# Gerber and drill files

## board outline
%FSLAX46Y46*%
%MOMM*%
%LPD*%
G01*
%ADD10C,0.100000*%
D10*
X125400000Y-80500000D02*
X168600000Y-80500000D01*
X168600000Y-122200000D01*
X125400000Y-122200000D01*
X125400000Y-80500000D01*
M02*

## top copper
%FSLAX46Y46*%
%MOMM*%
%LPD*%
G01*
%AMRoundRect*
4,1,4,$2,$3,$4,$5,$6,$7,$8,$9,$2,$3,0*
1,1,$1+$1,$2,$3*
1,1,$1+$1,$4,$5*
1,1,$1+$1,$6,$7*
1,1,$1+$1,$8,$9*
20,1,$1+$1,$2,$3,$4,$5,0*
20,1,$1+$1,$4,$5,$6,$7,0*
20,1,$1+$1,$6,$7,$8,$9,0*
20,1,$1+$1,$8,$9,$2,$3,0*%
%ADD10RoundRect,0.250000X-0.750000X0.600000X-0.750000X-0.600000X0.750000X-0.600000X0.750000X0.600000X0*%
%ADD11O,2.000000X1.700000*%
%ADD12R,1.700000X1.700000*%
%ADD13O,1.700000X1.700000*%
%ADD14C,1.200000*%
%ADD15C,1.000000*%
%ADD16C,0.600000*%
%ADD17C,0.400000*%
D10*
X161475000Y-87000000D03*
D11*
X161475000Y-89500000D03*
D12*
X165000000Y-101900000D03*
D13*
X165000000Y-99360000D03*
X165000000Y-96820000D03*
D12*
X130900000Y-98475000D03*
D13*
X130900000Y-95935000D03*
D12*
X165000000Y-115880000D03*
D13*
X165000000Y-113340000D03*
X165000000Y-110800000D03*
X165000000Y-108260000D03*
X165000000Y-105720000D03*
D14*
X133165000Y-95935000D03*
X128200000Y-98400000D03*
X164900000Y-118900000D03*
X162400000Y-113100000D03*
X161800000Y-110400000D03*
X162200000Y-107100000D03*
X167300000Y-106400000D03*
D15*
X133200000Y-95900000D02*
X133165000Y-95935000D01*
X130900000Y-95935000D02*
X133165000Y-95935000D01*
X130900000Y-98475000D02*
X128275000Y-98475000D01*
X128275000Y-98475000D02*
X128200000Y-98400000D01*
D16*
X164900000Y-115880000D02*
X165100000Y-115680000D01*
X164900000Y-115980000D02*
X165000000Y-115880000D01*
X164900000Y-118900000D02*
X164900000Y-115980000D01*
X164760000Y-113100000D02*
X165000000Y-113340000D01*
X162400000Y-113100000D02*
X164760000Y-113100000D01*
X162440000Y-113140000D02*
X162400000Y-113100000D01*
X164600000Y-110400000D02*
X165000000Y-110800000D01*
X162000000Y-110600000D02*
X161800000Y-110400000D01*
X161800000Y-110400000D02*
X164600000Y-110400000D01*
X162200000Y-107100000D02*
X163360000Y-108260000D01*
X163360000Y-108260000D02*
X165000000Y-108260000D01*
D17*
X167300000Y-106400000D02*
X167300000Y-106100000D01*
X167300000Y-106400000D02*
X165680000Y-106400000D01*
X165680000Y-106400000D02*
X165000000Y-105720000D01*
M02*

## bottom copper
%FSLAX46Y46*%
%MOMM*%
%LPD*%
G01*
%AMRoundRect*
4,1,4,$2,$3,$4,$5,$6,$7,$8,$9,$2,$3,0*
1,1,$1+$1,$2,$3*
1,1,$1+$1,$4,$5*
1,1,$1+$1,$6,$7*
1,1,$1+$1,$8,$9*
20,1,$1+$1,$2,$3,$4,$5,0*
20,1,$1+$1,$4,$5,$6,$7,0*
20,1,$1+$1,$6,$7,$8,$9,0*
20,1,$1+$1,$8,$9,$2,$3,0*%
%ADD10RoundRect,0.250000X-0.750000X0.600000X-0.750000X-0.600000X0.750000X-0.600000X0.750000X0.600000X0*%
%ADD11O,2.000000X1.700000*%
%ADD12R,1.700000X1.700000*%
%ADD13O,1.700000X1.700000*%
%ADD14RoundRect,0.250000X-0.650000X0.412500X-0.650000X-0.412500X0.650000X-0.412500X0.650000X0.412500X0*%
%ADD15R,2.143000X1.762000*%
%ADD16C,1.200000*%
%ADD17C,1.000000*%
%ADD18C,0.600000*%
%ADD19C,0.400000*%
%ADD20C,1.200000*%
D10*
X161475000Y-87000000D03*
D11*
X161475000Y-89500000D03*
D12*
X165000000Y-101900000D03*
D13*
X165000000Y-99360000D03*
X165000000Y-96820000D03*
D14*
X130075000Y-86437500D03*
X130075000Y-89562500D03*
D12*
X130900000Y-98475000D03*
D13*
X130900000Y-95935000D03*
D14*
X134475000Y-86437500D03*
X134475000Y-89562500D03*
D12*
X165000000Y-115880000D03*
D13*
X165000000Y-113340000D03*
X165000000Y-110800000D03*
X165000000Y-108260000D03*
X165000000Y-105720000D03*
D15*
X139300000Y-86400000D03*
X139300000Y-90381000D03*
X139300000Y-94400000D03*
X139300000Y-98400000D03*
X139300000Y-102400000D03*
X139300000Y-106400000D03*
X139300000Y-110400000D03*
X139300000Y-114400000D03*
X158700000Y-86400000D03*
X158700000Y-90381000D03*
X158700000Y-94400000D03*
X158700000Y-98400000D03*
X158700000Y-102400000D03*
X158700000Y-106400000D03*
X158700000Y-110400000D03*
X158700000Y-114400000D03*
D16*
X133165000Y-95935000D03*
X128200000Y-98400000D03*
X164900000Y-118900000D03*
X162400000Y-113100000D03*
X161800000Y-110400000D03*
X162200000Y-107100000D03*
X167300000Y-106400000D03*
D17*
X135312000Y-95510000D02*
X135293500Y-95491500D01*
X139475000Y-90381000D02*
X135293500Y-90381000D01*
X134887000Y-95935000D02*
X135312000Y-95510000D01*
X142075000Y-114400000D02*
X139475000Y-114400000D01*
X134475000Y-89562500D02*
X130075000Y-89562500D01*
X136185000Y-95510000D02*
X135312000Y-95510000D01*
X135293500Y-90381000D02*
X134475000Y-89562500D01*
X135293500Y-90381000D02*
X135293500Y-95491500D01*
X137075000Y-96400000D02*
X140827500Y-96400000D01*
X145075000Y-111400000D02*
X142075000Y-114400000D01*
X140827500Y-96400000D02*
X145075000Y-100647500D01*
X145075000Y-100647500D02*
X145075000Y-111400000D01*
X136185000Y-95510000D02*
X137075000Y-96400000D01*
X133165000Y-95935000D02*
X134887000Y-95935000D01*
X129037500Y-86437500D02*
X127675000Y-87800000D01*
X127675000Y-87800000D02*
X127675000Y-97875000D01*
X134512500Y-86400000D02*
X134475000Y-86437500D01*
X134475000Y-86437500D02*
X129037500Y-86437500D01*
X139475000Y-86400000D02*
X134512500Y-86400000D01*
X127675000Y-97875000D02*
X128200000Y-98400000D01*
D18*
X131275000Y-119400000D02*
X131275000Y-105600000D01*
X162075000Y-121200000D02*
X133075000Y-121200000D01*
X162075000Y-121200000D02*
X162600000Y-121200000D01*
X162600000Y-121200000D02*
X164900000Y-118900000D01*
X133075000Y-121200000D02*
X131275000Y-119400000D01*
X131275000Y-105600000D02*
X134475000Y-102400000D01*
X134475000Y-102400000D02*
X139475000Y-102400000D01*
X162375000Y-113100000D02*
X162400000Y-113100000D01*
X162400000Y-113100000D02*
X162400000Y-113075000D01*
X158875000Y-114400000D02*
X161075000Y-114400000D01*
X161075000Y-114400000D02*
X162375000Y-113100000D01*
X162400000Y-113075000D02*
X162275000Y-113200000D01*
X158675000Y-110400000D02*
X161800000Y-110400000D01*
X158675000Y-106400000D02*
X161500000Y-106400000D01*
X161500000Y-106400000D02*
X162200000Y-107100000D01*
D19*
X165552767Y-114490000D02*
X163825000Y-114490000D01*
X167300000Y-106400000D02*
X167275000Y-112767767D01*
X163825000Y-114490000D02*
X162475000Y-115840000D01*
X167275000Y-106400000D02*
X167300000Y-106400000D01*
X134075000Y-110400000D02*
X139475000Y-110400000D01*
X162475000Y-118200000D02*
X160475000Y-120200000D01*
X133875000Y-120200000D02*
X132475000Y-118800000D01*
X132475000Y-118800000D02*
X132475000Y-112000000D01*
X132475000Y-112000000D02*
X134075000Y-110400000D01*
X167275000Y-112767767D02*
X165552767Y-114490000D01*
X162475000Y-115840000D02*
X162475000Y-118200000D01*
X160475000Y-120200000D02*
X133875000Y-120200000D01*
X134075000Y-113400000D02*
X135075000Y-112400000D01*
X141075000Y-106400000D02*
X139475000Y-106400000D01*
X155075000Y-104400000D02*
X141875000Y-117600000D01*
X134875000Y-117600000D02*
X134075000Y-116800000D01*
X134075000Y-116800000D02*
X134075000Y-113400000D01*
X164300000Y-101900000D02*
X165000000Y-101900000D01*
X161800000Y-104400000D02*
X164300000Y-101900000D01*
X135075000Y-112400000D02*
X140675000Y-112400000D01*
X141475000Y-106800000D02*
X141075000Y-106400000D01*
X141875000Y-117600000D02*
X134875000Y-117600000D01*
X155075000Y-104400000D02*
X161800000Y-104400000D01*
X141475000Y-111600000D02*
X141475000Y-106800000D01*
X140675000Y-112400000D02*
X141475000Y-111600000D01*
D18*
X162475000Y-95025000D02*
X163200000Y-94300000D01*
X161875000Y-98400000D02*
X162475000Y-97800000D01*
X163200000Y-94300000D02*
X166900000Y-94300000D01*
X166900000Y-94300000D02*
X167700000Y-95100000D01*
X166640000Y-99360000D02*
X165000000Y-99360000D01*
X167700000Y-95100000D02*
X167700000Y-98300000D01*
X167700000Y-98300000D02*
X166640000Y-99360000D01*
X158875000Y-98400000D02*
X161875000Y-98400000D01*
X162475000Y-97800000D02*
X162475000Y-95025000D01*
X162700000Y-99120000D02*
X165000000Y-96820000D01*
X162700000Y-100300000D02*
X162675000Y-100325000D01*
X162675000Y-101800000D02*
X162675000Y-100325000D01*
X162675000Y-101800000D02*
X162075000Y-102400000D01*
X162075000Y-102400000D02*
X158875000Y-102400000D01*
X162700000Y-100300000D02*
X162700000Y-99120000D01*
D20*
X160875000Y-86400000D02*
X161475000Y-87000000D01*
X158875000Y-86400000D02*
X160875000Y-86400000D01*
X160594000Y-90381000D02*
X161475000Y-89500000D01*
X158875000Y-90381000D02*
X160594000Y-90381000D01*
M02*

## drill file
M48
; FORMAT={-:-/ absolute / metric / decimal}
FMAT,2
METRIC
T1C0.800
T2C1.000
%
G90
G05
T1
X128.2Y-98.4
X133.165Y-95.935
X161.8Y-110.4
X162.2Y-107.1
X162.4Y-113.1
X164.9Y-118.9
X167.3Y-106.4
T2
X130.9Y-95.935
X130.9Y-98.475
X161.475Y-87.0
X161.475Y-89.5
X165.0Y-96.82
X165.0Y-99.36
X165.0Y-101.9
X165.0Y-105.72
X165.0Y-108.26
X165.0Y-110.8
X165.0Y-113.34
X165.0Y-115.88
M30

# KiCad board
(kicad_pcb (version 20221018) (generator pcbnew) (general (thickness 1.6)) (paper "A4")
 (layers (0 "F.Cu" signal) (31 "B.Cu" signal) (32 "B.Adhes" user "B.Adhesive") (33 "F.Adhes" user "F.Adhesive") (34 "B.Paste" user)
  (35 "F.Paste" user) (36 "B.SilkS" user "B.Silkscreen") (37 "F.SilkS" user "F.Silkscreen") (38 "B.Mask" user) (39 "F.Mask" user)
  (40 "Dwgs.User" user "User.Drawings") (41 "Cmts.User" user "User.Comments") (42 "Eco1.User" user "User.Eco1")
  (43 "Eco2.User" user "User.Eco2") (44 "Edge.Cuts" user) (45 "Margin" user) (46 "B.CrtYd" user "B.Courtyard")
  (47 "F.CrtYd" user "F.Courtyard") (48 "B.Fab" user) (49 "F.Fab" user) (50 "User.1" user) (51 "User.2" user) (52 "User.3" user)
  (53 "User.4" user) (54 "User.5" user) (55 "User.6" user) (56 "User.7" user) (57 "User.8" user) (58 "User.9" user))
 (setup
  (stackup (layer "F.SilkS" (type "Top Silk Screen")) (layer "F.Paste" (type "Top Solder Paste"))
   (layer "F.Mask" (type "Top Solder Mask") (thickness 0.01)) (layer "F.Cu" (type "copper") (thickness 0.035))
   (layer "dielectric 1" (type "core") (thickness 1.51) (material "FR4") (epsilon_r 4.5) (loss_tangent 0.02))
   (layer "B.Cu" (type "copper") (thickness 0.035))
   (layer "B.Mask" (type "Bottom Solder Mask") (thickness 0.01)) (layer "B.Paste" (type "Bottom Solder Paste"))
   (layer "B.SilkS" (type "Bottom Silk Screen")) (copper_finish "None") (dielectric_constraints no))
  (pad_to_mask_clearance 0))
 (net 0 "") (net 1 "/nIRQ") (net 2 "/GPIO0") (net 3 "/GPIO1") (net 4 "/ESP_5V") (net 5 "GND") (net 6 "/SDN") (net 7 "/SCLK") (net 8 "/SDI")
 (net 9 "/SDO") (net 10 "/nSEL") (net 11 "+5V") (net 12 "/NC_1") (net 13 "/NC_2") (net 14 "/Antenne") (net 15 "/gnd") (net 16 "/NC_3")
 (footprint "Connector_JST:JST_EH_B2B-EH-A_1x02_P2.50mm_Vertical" (layer "F.Cu") (at 161.475 87 -90)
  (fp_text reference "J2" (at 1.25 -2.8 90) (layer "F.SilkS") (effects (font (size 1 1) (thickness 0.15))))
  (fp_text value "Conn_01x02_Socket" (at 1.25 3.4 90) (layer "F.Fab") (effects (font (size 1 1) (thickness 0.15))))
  (pad "1" thru_hole roundrect (at 0 0 270) (size 1.7 2) (drill 1) (layers "*.Cu" "*.Mask") (roundrect_rratio 0.1470588235))
  (pad "2" thru_hole oval (at 2.5 0 270) (size 1.7 2) (drill 1) (layers "*.Cu" "*.Mask")))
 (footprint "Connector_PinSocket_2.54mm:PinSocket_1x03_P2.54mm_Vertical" (layer "F.Cu") (at 165 101.9 180)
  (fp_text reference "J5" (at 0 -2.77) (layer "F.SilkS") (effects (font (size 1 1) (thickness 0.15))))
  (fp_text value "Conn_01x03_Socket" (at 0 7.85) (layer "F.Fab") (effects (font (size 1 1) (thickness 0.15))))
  (pad "1" thru_hole rect (at 0 0 180) (size 1.7 1.7) (drill 1) (layers "*.Cu" "*.Mask") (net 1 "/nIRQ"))
  (pad "2" thru_hole oval (at 0 2.54 180) (size 1.7 1.7) (drill 1) (layers "*.Cu" "*.Mask") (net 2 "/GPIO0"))
  (pad "3" thru_hole oval (at 0 5.08 180) (size 1.7 1.7) (drill 1) (layers "*.Cu" "*.Mask") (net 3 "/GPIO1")))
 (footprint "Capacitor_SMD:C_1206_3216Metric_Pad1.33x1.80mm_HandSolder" (layer "B.Cu") (at 130.075 88 -90)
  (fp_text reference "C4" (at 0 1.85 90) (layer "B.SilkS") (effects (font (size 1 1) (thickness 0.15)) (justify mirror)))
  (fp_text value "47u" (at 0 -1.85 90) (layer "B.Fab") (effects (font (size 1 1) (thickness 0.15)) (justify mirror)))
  (pad "1" smd roundrect (at -1.5625 0 270) (size 1.325 1.8) (layers "B.Cu" "B.Paste" "B.Mask") (roundrect_rratio 0.1886792453))
  (pad "2" smd roundrect (at 1.5625 0 270) (size 1.325 1.8) (layers "B.Cu" "B.Paste" "B.Mask") (roundrect_rratio 0.1886792453)))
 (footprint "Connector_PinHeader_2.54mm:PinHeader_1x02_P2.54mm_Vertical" (layer "B.Cu") (at 130.9 98.475)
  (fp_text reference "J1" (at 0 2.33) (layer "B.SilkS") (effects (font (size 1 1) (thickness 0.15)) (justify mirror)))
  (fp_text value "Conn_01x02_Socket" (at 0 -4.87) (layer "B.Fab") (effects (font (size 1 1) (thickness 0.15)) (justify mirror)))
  (pad "1" thru_hole rect (at 0 0) (size 1.7 1.7) (drill 1) (layers "*.Cu" "*.Mask") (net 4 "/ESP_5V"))
  (pad "2" thru_hole oval (at 0 -2.54) (size 1.7 1.7) (drill 1) (layers "*.Cu" "*.Mask") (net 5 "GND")))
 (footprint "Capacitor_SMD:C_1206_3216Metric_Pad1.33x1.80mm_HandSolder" (layer "B.Cu") (at 134.475 88 -90)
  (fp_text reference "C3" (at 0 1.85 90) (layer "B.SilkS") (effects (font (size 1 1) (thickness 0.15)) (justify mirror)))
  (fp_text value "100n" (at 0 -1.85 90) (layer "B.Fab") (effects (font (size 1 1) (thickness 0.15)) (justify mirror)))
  (pad "1" smd roundrect (at -1.5625 0 270) (size 1.325 1.8) (layers "B.Cu" "B.Paste" "B.Mask") (roundrect_rratio 0.1886792453))
  (pad "2" smd roundrect (at 1.5625 0 270) (size 1.325 1.8) (layers "B.Cu" "B.Paste" "B.Mask") (roundrect_rratio 0.1886792453)))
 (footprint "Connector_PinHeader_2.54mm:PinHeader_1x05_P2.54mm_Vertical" (layer "B.Cu") (at 165 115.88)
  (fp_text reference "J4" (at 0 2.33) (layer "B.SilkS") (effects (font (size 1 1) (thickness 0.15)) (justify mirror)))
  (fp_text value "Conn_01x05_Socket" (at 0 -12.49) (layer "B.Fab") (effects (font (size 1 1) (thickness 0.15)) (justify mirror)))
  (pad "1" thru_hole rect (at 0 0) (size 1.7 1.7) (drill 1) (layers "*.Cu" "*.Mask") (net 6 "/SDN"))
  (pad "2" thru_hole oval (at 0 -2.54) (size 1.7 1.7) (drill 1) (layers "*.Cu" "*.Mask") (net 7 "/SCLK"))
  (pad "3" thru_hole oval (at 0 -5.08) (size 1.7 1.7) (drill 1) (layers "*.Cu" "*.Mask") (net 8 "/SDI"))
  (pad "4" thru_hole oval (at 0 -7.62) (size 1.7 1.7) (drill 1) (layers "*.Cu" "*.Mask") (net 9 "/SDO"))
  (pad "5" thru_hole oval (at 0 -10.16) (size 1.7 1.7) (drill 1) (layers "*.Cu" "*.Mask") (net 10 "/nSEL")))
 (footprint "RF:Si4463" (layer "B.Cu") (at 149 100.4 -90)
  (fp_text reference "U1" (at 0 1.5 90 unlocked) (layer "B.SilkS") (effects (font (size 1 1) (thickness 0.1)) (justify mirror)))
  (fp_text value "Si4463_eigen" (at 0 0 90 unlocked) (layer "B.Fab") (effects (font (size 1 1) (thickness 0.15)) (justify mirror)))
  (pad "1" smd rect (at -14 9.7 180) (size 2.143 1.762) (layers "B.Cu" "B.Paste" "B.Mask") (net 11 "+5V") (thermal_bridge_angle 45))
  (pad "2" smd rect (at -10.019 9.7 180) (size 2.143 1.762) (layers "B.Cu" "B.Paste" "B.Mask") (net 5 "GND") (thermal_bridge_angle 45))
  (pad "3" smd rect (at -6 9.7 180) (size 2.143 1.762) (layers "B.Cu" "B.Paste" "B.Mask") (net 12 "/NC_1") (thermal_bridge_angle 45))
  (pad "4" smd rect (at -2 9.7 180) (size 2.143 1.762) (layers "B.Cu" "B.Paste" "B.Mask") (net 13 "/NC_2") (thermal_bridge_angle 45))
  (pad "5" smd rect (at 2 9.7 180) (size 2.143 1.762) (layers "B.Cu" "B.Paste" "B.Mask") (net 6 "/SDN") (thermal_bridge_angle 45))
  (pad "6" smd rect (at 6 9.7 180) (size 2.143 1.762) (layers "B.Cu" "B.Paste" "B.Mask") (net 1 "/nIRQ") (thermal_bridge_angle 45))
  (pad "7" smd rect (at 10 9.7 180) (size 2.143 1.762) (layers "B.Cu" "B.Paste" "B.Mask") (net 10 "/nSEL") (thermal_bridge_angle 45))
  (pad "8" smd rect (at 14 9.7 180) (size 2.143 1.762) (layers "B.Cu" "B.Paste" "B.Mask") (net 5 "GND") (thermal_bridge_angle 45))
  (pad "9" smd rect (at -14 -9.7 180) (size 2.143 1.762) (layers "B.Cu" "B.Paste" "B.Mask") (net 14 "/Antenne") (thermal_bridge_angle 45))
  (pad "10" smd rect (at -10.019 -9.7 180) (size 2.143 1.762) (layers "B.Cu" "B.Paste" "B.Mask") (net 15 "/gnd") (thermal_bridge_angle 45))
  (pad "11" smd rect (at -6 -9.7 180) (size 2.143 1.762) (layers "B.Cu" "B.Paste" "B.Mask") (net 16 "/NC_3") (thermal_bridge_angle 45))
  (pad "12" smd rect (at -2 -9.7 180) (size 2.143 1.762) (layers "B.Cu" "B.Paste" "B.Mask") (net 2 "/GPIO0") (thermal_bridge_angle 45))
  (pad "13" smd rect (at 2 -9.7 180) (size 2.143 1.762) (layers "B.Cu" "B.Paste" "B.Mask") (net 3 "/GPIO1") (thermal_bridge_angle 45))
  (pad "14" smd rect (at 6 -9.7 180) (size 2.143 1.762) (layers "B.Cu" "B.Paste" "B.Mask") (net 9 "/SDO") (thermal_bridge_angle 45))
  (pad "15" smd rect (at 10 -9.7 180) (size 2.143 1.762) (layers "B.Cu" "B.Paste" "B.Mask") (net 8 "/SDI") (thermal_bridge_angle 45))
  (pad "16" smd rect (at 14 -9.7 180) (size 2.143 1.762) (layers "B.Cu" "B.Paste" "B.Mask") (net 7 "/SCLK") (thermal_bridge_angle 45)))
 (gr_rect (start 125.4 80.5) (end 168.6 122.2) (stroke (width 0.1) (type default)) (fill none) (layer "Edge.Cuts"))
 (segment (start 133.2 95.9) (end 133.165 95.935) (width 1) (layer "F.Cu") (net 5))
 (segment (start 130.9 95.935) (end 133.165 95.935) (width 1) (layer "F.Cu") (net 5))
 (via (at 133.165 95.935) (size 1.2) (drill 0.8) (layers "F.Cu" "B.Cu") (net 5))
 (segment (start 135.312 95.51) (end 135.2935 95.4915) (width 1) (layer "B.Cu") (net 5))
 (segment (start 139.475 90.381) (end 135.2935 90.381) (width 1) (layer "B.Cu") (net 5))
 (segment (start 134.887 95.935) (end 135.312 95.51) (width 1) (layer "B.Cu") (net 5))
 (segment (start 142.075 114.4) (end 139.475 114.4) (width 1) (layer "B.Cu") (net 5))
 (segment (start 134.475 89.5625) (end 130.075 89.5625) (width 1) (layer "B.Cu") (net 5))
 (segment (start 136.185 95.51) (end 135.312 95.51) (width 1) (layer "B.Cu") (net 5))
 (segment (start 135.2935 90.381) (end 134.475 89.5625) (width 1) (layer "B.Cu") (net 5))
 (segment (start 135.2935 90.381) (end 135.2935 95.4915) (width 1) (layer "B.Cu") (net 5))
 (segment (start 137.075 96.4) (end 140.8275 96.4) (width 1) (layer "B.Cu") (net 5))
 (segment (start 145.075 111.4) (end 142.075 114.4) (width 1) (layer "B.Cu") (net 5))
 (segment (start 140.8275 96.4) (end 145.075 100.6475) (width 1) (layer "B.Cu") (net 5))
 (segment (start 145.075 100.6475) (end 145.075 111.4) (width 1) (layer "B.Cu") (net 5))
 (segment (start 136.185 95.51) (end 137.075 96.4) (width 1) (layer "B.Cu") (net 5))
 (segment (start 133.165 95.935) (end 134.887 95.935) (width 1) (layer "B.Cu") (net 5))
 (segment (start 130.9 98.475) (end 128.275 98.475) (width 1) (layer "F.Cu") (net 4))
 (segment (start 128.275 98.475) (end 128.2 98.4) (width 1) (layer "F.Cu") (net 4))
 (via (at 128.2 98.4) (size 1.2) (drill 0.8) (layers "F.Cu" "B.Cu") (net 4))
 (segment (start 129.0375 86.4375) (end 127.675 87.8) (width 1) (layer "B.Cu") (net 4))
 (segment (start 127.675 87.8) (end 127.675 97.875) (width 1) (layer "B.Cu") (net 4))
 (segment (start 134.5125 86.4) (end 134.475 86.4375) (width 1) (layer "B.Cu") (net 4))
 (segment (start 134.475 86.4375) (end 129.0375 86.4375) (width 1) (layer "B.Cu") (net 4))
 (segment (start 139.475 86.4) (end 134.5125 86.4) (width 1) (layer "B.Cu") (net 4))
 (segment (start 127.675 97.875) (end 128.2 98.4) (width 1) (layer "B.Cu") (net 4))
 (segment (start 164.9 115.88) (end 165.1 115.68) (width 0.6) (layer "F.Cu") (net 6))
 (segment (start 164.9 115.98) (end 165 115.88) (width 0.6) (layer "F.Cu") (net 6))
 (segment (start 164.9 118.9) (end 164.9 115.98) (width 0.6) (layer "F.Cu") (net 6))
 (via (at 164.9 118.9) (size 1.2) (drill 0.8) (layers "F.Cu" "B.Cu") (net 6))
 (segment (start 131.275 119.4) (end 131.275 105.6) (width 0.6) (layer "B.Cu") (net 6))
 (segment (start 162.075 121.2) (end 133.075 121.2) (width 0.6) (layer "B.Cu") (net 6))
 (segment (start 162.075 121.2) (end 162.6 121.2) (width 0.6) (layer "B.Cu") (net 6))
 (segment (start 162.6 121.2) (end 164.9 118.9) (width 0.6) (layer "B.Cu") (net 6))
 (segment (start 133.075 121.2) (end 131.275 119.4) (width 0.6) (layer "B.Cu") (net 6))
 (segment (start 131.275 105.6) (end 134.475 102.4) (width 0.6) (layer "B.Cu") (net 6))
 (segment (start 134.475 102.4) (end 139.475 102.4) (width 0.6) (layer "B.Cu") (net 6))
 (segment (start 164.76 113.1) (end 165 113.34) (width 0.6) (layer "F.Cu") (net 7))
 (segment (start 162.4 113.1) (end 164.76 113.1) (width 0.6) (layer "F.Cu") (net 7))
 (segment (start 162.44 113.14) (end 162.4 113.1) (width 0.6) (layer "F.Cu") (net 7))
 (via (at 162.4 113.1) (size 1.2) (drill 0.8) (layers "F.Cu" "B.Cu") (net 7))
 (segment (start 162.375 113.1) (end 162.4 113.1) (width 0.6) (layer "B.Cu") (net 7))
 (segment (start 162.4 113.1) (end 162.4 113.075) (width 0.6) (layer "B.Cu") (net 7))
 (segment (start 158.875 114.4) (end 161.075 114.4) (width 0.6) (layer "B.Cu") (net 7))
 (segment (start 161.075 114.4) (end 162.375 113.1) (width 0.6) (layer "B.Cu") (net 7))
 (segment (start 162.4 113.075) (end 162.275 113.2) (width 0.6) (layer "B.Cu") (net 7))
 (segment (start 164.6 110.4) (end 165 110.8) (width 0.6) (layer "F.Cu") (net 8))
 (segment (start 162 110.6) (end 161.8 110.4) (width 0.6) (layer "F.Cu") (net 8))
 (segment (start 161.8 110.4) (end 164.6 110.4) (width 0.6) (layer "F.Cu") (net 8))
 (via (at 161.8 110.4) (size 1.2) (drill 0.8) (layers "F.Cu" "B.Cu") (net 8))
 (segment (start 158.675 110.4) (end 161.8 110.4) (width 0.6) (layer "B.Cu") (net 8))
 (segment (start 162.2 107.1) (end 163.36 108.26) (width 0.6) (layer "F.Cu") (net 9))
 (segment (start 163.36 108.26) (end 165 108.26) (width 0.6) (layer "F.Cu") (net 9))
 (via (at 162.2 107.1) (size 1.2) (drill 0.8) (layers "F.Cu" "B.Cu") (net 9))
 (segment (start 158.675 106.4) (end 161.5 106.4) (width 0.6) (layer "B.Cu") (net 9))
 (segment (start 161.5 106.4) (end 162.2 107.1) (width 0.6) (layer "B.Cu") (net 9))
 (segment (start 167.3 106.4) (end 167.3 106.1) (width 0.4) (layer "F.Cu") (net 10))
 (segment (start 167.3 106.4) (end 165.68 106.4) (width 0.4) (layer "F.Cu") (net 10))
 (segment (start 165.68 106.4) (end 165 105.72) (width 0.4) (layer "F.Cu") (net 10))
 (via (at 167.3 106.4) (size 1.2) (drill 0.8) (layers "F.Cu" "B.Cu") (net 10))
 (segment (start 165.552767 114.49) (end 163.825 114.49) (width 0.4) (layer "B.Cu") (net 10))
 (segment (start 167.3 106.4) (end 167.275 112.767767) (width 0.4) (layer "B.Cu") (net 10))
 (segment (start 163.825 114.49) (end 162.475 115.84) (width 0.4) (layer "B.Cu") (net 10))
 (segment (start 167.275 106.4) (end 167.3 106.4) (width 0.4) (layer "B.Cu") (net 10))
 (segment (start 134.075 110.4) (end 139.475 110.4) (width 0.4) (layer "B.Cu") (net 10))
 (segment (start 162.475 118.2) (end 160.475 120.2) (width 0.4) (layer "B.Cu") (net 10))
 (segment (start 133.875 120.2) (end 132.475 118.8) (width 0.4) (layer "B.Cu") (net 10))
 (segment (start 132.475 118.8) (end 132.475 112) (width 0.4) (layer "B.Cu") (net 10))
 (segment (start 132.475 112) (end 134.075 110.4) (width 0.4) (layer "B.Cu") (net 10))
 (segment (start 167.275 112.767767) (end 165.552767 114.49) (width 0.4) (layer "B.Cu") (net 10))
 (segment (start 162.475 115.84) (end 162.475 118.2) (width 0.4) (layer "B.Cu") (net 10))
 (segment (start 160.475 120.2) (end 133.875 120.2) (width 0.4) (layer "B.Cu") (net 10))
 (segment (start 134.075 113.4) (end 135.075 112.4) (width 0.4) (layer "B.Cu") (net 1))
 (segment (start 141.075 106.4) (end 139.475 106.4) (width 0.4) (layer "B.Cu") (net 1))
 (segment (start 155.075 104.4) (end 141.875 117.6) (width 0.4) (layer "B.Cu") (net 1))
 (segment (start 134.875 117.6) (end 134.075 116.8) (width 0.4) (layer "B.Cu") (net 1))
 (segment (start 134.075 116.8) (end 134.075 113.4) (width 0.4) (layer "B.Cu") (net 1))
 (segment (start 164.3 101.9) (end 165 101.9) (width 0.4) (layer "B.Cu") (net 1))
 (segment (start 161.8 104.4) (end 164.3 101.9) (width 0.4) (layer "B.Cu") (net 1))
 (segment (start 135.075 112.4) (end 140.675 112.4) (width 0.4) (layer "B.Cu") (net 1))
 (segment (start 141.475 106.8) (end 141.075 106.4) (width 0.4) (layer "B.Cu") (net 1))
 (segment (start 141.875 117.6) (end 134.875 117.6) (width 0.4) (layer "B.Cu") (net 1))
 (segment (start 155.075 104.4) (end 161.8 104.4) (width 0.4) (layer "B.Cu") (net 1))
 (segment (start 141.475 111.6) (end 141.475 106.8) (width 0.4) (layer "B.Cu") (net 1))
 (segment (start 140.675 112.4) (end 141.475 111.6) (width 0.4) (layer "B.Cu") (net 1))
 (segment (start 162.475 95.025) (end 163.2 94.3) (width 0.6) (layer "B.Cu") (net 2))
 (segment (start 161.875 98.4) (end 162.475 97.8) (width 0.6) (layer "B.Cu") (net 2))
 (segment (start 163.2 94.3) (end 166.9 94.3) (width 0.6) (layer "B.Cu") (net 2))
 (segment (start 166.9 94.3) (end 167.7 95.1) (width 0.6) (layer "B.Cu") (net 2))
 (segment (start 166.64 99.36) (end 165 99.36) (width 0.6) (layer "B.Cu") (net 2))
 (segment (start 167.7 95.1) (end 167.7 98.3) (width 0.6) (layer "B.Cu") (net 2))
 (segment (start 167.7 98.3) (end 166.64 99.36) (width 0.6) (layer "B.Cu") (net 2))
 (segment (start 158.875 98.4) (end 161.875 98.4) (width 0.6) (layer "B.Cu") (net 2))
 (segment (start 162.475 97.8) (end 162.475 95.025) (width 0.6) (layer "B.Cu") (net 2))
 (segment (start 162.7 99.12) (end 165 96.82) (width 0.6) (layer "B.Cu") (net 3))
 (segment (start 162.7 100.3) (end 162.675 100.325) (width 0.6) (layer "B.Cu") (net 3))
 (segment (start 162.675 101.8) (end 162.675 100.325) (width 0.6) (layer "B.Cu") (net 3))
 (segment (start 162.675 101.8) (end 162.075 102.4) (width 0.6) (layer "B.Cu") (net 3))
 (segment (start 162.075 102.4) (end 158.875 102.4) (width 0.6) (layer "B.Cu") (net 3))
 (segment (start 162.7 100.3) (end 162.7 99.12) (width 0.6) (layer "B.Cu") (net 3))
 (segment (start 160.875 86.4) (end 161.475 87) (width 1.2) (layer "B.Cu") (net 14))
 (segment (start 158.875 86.4) (end 160.875 86.4) (width 1.2) (layer "B.Cu") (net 14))
 (segment (start 160.594 90.381) (end 161.475 89.5) (width 1.2) (layer "B.Cu") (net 15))
 (segment (start 158.875 90.381) (end 160.594 90.381) (width 1.2) (layer "B.Cu") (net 15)))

